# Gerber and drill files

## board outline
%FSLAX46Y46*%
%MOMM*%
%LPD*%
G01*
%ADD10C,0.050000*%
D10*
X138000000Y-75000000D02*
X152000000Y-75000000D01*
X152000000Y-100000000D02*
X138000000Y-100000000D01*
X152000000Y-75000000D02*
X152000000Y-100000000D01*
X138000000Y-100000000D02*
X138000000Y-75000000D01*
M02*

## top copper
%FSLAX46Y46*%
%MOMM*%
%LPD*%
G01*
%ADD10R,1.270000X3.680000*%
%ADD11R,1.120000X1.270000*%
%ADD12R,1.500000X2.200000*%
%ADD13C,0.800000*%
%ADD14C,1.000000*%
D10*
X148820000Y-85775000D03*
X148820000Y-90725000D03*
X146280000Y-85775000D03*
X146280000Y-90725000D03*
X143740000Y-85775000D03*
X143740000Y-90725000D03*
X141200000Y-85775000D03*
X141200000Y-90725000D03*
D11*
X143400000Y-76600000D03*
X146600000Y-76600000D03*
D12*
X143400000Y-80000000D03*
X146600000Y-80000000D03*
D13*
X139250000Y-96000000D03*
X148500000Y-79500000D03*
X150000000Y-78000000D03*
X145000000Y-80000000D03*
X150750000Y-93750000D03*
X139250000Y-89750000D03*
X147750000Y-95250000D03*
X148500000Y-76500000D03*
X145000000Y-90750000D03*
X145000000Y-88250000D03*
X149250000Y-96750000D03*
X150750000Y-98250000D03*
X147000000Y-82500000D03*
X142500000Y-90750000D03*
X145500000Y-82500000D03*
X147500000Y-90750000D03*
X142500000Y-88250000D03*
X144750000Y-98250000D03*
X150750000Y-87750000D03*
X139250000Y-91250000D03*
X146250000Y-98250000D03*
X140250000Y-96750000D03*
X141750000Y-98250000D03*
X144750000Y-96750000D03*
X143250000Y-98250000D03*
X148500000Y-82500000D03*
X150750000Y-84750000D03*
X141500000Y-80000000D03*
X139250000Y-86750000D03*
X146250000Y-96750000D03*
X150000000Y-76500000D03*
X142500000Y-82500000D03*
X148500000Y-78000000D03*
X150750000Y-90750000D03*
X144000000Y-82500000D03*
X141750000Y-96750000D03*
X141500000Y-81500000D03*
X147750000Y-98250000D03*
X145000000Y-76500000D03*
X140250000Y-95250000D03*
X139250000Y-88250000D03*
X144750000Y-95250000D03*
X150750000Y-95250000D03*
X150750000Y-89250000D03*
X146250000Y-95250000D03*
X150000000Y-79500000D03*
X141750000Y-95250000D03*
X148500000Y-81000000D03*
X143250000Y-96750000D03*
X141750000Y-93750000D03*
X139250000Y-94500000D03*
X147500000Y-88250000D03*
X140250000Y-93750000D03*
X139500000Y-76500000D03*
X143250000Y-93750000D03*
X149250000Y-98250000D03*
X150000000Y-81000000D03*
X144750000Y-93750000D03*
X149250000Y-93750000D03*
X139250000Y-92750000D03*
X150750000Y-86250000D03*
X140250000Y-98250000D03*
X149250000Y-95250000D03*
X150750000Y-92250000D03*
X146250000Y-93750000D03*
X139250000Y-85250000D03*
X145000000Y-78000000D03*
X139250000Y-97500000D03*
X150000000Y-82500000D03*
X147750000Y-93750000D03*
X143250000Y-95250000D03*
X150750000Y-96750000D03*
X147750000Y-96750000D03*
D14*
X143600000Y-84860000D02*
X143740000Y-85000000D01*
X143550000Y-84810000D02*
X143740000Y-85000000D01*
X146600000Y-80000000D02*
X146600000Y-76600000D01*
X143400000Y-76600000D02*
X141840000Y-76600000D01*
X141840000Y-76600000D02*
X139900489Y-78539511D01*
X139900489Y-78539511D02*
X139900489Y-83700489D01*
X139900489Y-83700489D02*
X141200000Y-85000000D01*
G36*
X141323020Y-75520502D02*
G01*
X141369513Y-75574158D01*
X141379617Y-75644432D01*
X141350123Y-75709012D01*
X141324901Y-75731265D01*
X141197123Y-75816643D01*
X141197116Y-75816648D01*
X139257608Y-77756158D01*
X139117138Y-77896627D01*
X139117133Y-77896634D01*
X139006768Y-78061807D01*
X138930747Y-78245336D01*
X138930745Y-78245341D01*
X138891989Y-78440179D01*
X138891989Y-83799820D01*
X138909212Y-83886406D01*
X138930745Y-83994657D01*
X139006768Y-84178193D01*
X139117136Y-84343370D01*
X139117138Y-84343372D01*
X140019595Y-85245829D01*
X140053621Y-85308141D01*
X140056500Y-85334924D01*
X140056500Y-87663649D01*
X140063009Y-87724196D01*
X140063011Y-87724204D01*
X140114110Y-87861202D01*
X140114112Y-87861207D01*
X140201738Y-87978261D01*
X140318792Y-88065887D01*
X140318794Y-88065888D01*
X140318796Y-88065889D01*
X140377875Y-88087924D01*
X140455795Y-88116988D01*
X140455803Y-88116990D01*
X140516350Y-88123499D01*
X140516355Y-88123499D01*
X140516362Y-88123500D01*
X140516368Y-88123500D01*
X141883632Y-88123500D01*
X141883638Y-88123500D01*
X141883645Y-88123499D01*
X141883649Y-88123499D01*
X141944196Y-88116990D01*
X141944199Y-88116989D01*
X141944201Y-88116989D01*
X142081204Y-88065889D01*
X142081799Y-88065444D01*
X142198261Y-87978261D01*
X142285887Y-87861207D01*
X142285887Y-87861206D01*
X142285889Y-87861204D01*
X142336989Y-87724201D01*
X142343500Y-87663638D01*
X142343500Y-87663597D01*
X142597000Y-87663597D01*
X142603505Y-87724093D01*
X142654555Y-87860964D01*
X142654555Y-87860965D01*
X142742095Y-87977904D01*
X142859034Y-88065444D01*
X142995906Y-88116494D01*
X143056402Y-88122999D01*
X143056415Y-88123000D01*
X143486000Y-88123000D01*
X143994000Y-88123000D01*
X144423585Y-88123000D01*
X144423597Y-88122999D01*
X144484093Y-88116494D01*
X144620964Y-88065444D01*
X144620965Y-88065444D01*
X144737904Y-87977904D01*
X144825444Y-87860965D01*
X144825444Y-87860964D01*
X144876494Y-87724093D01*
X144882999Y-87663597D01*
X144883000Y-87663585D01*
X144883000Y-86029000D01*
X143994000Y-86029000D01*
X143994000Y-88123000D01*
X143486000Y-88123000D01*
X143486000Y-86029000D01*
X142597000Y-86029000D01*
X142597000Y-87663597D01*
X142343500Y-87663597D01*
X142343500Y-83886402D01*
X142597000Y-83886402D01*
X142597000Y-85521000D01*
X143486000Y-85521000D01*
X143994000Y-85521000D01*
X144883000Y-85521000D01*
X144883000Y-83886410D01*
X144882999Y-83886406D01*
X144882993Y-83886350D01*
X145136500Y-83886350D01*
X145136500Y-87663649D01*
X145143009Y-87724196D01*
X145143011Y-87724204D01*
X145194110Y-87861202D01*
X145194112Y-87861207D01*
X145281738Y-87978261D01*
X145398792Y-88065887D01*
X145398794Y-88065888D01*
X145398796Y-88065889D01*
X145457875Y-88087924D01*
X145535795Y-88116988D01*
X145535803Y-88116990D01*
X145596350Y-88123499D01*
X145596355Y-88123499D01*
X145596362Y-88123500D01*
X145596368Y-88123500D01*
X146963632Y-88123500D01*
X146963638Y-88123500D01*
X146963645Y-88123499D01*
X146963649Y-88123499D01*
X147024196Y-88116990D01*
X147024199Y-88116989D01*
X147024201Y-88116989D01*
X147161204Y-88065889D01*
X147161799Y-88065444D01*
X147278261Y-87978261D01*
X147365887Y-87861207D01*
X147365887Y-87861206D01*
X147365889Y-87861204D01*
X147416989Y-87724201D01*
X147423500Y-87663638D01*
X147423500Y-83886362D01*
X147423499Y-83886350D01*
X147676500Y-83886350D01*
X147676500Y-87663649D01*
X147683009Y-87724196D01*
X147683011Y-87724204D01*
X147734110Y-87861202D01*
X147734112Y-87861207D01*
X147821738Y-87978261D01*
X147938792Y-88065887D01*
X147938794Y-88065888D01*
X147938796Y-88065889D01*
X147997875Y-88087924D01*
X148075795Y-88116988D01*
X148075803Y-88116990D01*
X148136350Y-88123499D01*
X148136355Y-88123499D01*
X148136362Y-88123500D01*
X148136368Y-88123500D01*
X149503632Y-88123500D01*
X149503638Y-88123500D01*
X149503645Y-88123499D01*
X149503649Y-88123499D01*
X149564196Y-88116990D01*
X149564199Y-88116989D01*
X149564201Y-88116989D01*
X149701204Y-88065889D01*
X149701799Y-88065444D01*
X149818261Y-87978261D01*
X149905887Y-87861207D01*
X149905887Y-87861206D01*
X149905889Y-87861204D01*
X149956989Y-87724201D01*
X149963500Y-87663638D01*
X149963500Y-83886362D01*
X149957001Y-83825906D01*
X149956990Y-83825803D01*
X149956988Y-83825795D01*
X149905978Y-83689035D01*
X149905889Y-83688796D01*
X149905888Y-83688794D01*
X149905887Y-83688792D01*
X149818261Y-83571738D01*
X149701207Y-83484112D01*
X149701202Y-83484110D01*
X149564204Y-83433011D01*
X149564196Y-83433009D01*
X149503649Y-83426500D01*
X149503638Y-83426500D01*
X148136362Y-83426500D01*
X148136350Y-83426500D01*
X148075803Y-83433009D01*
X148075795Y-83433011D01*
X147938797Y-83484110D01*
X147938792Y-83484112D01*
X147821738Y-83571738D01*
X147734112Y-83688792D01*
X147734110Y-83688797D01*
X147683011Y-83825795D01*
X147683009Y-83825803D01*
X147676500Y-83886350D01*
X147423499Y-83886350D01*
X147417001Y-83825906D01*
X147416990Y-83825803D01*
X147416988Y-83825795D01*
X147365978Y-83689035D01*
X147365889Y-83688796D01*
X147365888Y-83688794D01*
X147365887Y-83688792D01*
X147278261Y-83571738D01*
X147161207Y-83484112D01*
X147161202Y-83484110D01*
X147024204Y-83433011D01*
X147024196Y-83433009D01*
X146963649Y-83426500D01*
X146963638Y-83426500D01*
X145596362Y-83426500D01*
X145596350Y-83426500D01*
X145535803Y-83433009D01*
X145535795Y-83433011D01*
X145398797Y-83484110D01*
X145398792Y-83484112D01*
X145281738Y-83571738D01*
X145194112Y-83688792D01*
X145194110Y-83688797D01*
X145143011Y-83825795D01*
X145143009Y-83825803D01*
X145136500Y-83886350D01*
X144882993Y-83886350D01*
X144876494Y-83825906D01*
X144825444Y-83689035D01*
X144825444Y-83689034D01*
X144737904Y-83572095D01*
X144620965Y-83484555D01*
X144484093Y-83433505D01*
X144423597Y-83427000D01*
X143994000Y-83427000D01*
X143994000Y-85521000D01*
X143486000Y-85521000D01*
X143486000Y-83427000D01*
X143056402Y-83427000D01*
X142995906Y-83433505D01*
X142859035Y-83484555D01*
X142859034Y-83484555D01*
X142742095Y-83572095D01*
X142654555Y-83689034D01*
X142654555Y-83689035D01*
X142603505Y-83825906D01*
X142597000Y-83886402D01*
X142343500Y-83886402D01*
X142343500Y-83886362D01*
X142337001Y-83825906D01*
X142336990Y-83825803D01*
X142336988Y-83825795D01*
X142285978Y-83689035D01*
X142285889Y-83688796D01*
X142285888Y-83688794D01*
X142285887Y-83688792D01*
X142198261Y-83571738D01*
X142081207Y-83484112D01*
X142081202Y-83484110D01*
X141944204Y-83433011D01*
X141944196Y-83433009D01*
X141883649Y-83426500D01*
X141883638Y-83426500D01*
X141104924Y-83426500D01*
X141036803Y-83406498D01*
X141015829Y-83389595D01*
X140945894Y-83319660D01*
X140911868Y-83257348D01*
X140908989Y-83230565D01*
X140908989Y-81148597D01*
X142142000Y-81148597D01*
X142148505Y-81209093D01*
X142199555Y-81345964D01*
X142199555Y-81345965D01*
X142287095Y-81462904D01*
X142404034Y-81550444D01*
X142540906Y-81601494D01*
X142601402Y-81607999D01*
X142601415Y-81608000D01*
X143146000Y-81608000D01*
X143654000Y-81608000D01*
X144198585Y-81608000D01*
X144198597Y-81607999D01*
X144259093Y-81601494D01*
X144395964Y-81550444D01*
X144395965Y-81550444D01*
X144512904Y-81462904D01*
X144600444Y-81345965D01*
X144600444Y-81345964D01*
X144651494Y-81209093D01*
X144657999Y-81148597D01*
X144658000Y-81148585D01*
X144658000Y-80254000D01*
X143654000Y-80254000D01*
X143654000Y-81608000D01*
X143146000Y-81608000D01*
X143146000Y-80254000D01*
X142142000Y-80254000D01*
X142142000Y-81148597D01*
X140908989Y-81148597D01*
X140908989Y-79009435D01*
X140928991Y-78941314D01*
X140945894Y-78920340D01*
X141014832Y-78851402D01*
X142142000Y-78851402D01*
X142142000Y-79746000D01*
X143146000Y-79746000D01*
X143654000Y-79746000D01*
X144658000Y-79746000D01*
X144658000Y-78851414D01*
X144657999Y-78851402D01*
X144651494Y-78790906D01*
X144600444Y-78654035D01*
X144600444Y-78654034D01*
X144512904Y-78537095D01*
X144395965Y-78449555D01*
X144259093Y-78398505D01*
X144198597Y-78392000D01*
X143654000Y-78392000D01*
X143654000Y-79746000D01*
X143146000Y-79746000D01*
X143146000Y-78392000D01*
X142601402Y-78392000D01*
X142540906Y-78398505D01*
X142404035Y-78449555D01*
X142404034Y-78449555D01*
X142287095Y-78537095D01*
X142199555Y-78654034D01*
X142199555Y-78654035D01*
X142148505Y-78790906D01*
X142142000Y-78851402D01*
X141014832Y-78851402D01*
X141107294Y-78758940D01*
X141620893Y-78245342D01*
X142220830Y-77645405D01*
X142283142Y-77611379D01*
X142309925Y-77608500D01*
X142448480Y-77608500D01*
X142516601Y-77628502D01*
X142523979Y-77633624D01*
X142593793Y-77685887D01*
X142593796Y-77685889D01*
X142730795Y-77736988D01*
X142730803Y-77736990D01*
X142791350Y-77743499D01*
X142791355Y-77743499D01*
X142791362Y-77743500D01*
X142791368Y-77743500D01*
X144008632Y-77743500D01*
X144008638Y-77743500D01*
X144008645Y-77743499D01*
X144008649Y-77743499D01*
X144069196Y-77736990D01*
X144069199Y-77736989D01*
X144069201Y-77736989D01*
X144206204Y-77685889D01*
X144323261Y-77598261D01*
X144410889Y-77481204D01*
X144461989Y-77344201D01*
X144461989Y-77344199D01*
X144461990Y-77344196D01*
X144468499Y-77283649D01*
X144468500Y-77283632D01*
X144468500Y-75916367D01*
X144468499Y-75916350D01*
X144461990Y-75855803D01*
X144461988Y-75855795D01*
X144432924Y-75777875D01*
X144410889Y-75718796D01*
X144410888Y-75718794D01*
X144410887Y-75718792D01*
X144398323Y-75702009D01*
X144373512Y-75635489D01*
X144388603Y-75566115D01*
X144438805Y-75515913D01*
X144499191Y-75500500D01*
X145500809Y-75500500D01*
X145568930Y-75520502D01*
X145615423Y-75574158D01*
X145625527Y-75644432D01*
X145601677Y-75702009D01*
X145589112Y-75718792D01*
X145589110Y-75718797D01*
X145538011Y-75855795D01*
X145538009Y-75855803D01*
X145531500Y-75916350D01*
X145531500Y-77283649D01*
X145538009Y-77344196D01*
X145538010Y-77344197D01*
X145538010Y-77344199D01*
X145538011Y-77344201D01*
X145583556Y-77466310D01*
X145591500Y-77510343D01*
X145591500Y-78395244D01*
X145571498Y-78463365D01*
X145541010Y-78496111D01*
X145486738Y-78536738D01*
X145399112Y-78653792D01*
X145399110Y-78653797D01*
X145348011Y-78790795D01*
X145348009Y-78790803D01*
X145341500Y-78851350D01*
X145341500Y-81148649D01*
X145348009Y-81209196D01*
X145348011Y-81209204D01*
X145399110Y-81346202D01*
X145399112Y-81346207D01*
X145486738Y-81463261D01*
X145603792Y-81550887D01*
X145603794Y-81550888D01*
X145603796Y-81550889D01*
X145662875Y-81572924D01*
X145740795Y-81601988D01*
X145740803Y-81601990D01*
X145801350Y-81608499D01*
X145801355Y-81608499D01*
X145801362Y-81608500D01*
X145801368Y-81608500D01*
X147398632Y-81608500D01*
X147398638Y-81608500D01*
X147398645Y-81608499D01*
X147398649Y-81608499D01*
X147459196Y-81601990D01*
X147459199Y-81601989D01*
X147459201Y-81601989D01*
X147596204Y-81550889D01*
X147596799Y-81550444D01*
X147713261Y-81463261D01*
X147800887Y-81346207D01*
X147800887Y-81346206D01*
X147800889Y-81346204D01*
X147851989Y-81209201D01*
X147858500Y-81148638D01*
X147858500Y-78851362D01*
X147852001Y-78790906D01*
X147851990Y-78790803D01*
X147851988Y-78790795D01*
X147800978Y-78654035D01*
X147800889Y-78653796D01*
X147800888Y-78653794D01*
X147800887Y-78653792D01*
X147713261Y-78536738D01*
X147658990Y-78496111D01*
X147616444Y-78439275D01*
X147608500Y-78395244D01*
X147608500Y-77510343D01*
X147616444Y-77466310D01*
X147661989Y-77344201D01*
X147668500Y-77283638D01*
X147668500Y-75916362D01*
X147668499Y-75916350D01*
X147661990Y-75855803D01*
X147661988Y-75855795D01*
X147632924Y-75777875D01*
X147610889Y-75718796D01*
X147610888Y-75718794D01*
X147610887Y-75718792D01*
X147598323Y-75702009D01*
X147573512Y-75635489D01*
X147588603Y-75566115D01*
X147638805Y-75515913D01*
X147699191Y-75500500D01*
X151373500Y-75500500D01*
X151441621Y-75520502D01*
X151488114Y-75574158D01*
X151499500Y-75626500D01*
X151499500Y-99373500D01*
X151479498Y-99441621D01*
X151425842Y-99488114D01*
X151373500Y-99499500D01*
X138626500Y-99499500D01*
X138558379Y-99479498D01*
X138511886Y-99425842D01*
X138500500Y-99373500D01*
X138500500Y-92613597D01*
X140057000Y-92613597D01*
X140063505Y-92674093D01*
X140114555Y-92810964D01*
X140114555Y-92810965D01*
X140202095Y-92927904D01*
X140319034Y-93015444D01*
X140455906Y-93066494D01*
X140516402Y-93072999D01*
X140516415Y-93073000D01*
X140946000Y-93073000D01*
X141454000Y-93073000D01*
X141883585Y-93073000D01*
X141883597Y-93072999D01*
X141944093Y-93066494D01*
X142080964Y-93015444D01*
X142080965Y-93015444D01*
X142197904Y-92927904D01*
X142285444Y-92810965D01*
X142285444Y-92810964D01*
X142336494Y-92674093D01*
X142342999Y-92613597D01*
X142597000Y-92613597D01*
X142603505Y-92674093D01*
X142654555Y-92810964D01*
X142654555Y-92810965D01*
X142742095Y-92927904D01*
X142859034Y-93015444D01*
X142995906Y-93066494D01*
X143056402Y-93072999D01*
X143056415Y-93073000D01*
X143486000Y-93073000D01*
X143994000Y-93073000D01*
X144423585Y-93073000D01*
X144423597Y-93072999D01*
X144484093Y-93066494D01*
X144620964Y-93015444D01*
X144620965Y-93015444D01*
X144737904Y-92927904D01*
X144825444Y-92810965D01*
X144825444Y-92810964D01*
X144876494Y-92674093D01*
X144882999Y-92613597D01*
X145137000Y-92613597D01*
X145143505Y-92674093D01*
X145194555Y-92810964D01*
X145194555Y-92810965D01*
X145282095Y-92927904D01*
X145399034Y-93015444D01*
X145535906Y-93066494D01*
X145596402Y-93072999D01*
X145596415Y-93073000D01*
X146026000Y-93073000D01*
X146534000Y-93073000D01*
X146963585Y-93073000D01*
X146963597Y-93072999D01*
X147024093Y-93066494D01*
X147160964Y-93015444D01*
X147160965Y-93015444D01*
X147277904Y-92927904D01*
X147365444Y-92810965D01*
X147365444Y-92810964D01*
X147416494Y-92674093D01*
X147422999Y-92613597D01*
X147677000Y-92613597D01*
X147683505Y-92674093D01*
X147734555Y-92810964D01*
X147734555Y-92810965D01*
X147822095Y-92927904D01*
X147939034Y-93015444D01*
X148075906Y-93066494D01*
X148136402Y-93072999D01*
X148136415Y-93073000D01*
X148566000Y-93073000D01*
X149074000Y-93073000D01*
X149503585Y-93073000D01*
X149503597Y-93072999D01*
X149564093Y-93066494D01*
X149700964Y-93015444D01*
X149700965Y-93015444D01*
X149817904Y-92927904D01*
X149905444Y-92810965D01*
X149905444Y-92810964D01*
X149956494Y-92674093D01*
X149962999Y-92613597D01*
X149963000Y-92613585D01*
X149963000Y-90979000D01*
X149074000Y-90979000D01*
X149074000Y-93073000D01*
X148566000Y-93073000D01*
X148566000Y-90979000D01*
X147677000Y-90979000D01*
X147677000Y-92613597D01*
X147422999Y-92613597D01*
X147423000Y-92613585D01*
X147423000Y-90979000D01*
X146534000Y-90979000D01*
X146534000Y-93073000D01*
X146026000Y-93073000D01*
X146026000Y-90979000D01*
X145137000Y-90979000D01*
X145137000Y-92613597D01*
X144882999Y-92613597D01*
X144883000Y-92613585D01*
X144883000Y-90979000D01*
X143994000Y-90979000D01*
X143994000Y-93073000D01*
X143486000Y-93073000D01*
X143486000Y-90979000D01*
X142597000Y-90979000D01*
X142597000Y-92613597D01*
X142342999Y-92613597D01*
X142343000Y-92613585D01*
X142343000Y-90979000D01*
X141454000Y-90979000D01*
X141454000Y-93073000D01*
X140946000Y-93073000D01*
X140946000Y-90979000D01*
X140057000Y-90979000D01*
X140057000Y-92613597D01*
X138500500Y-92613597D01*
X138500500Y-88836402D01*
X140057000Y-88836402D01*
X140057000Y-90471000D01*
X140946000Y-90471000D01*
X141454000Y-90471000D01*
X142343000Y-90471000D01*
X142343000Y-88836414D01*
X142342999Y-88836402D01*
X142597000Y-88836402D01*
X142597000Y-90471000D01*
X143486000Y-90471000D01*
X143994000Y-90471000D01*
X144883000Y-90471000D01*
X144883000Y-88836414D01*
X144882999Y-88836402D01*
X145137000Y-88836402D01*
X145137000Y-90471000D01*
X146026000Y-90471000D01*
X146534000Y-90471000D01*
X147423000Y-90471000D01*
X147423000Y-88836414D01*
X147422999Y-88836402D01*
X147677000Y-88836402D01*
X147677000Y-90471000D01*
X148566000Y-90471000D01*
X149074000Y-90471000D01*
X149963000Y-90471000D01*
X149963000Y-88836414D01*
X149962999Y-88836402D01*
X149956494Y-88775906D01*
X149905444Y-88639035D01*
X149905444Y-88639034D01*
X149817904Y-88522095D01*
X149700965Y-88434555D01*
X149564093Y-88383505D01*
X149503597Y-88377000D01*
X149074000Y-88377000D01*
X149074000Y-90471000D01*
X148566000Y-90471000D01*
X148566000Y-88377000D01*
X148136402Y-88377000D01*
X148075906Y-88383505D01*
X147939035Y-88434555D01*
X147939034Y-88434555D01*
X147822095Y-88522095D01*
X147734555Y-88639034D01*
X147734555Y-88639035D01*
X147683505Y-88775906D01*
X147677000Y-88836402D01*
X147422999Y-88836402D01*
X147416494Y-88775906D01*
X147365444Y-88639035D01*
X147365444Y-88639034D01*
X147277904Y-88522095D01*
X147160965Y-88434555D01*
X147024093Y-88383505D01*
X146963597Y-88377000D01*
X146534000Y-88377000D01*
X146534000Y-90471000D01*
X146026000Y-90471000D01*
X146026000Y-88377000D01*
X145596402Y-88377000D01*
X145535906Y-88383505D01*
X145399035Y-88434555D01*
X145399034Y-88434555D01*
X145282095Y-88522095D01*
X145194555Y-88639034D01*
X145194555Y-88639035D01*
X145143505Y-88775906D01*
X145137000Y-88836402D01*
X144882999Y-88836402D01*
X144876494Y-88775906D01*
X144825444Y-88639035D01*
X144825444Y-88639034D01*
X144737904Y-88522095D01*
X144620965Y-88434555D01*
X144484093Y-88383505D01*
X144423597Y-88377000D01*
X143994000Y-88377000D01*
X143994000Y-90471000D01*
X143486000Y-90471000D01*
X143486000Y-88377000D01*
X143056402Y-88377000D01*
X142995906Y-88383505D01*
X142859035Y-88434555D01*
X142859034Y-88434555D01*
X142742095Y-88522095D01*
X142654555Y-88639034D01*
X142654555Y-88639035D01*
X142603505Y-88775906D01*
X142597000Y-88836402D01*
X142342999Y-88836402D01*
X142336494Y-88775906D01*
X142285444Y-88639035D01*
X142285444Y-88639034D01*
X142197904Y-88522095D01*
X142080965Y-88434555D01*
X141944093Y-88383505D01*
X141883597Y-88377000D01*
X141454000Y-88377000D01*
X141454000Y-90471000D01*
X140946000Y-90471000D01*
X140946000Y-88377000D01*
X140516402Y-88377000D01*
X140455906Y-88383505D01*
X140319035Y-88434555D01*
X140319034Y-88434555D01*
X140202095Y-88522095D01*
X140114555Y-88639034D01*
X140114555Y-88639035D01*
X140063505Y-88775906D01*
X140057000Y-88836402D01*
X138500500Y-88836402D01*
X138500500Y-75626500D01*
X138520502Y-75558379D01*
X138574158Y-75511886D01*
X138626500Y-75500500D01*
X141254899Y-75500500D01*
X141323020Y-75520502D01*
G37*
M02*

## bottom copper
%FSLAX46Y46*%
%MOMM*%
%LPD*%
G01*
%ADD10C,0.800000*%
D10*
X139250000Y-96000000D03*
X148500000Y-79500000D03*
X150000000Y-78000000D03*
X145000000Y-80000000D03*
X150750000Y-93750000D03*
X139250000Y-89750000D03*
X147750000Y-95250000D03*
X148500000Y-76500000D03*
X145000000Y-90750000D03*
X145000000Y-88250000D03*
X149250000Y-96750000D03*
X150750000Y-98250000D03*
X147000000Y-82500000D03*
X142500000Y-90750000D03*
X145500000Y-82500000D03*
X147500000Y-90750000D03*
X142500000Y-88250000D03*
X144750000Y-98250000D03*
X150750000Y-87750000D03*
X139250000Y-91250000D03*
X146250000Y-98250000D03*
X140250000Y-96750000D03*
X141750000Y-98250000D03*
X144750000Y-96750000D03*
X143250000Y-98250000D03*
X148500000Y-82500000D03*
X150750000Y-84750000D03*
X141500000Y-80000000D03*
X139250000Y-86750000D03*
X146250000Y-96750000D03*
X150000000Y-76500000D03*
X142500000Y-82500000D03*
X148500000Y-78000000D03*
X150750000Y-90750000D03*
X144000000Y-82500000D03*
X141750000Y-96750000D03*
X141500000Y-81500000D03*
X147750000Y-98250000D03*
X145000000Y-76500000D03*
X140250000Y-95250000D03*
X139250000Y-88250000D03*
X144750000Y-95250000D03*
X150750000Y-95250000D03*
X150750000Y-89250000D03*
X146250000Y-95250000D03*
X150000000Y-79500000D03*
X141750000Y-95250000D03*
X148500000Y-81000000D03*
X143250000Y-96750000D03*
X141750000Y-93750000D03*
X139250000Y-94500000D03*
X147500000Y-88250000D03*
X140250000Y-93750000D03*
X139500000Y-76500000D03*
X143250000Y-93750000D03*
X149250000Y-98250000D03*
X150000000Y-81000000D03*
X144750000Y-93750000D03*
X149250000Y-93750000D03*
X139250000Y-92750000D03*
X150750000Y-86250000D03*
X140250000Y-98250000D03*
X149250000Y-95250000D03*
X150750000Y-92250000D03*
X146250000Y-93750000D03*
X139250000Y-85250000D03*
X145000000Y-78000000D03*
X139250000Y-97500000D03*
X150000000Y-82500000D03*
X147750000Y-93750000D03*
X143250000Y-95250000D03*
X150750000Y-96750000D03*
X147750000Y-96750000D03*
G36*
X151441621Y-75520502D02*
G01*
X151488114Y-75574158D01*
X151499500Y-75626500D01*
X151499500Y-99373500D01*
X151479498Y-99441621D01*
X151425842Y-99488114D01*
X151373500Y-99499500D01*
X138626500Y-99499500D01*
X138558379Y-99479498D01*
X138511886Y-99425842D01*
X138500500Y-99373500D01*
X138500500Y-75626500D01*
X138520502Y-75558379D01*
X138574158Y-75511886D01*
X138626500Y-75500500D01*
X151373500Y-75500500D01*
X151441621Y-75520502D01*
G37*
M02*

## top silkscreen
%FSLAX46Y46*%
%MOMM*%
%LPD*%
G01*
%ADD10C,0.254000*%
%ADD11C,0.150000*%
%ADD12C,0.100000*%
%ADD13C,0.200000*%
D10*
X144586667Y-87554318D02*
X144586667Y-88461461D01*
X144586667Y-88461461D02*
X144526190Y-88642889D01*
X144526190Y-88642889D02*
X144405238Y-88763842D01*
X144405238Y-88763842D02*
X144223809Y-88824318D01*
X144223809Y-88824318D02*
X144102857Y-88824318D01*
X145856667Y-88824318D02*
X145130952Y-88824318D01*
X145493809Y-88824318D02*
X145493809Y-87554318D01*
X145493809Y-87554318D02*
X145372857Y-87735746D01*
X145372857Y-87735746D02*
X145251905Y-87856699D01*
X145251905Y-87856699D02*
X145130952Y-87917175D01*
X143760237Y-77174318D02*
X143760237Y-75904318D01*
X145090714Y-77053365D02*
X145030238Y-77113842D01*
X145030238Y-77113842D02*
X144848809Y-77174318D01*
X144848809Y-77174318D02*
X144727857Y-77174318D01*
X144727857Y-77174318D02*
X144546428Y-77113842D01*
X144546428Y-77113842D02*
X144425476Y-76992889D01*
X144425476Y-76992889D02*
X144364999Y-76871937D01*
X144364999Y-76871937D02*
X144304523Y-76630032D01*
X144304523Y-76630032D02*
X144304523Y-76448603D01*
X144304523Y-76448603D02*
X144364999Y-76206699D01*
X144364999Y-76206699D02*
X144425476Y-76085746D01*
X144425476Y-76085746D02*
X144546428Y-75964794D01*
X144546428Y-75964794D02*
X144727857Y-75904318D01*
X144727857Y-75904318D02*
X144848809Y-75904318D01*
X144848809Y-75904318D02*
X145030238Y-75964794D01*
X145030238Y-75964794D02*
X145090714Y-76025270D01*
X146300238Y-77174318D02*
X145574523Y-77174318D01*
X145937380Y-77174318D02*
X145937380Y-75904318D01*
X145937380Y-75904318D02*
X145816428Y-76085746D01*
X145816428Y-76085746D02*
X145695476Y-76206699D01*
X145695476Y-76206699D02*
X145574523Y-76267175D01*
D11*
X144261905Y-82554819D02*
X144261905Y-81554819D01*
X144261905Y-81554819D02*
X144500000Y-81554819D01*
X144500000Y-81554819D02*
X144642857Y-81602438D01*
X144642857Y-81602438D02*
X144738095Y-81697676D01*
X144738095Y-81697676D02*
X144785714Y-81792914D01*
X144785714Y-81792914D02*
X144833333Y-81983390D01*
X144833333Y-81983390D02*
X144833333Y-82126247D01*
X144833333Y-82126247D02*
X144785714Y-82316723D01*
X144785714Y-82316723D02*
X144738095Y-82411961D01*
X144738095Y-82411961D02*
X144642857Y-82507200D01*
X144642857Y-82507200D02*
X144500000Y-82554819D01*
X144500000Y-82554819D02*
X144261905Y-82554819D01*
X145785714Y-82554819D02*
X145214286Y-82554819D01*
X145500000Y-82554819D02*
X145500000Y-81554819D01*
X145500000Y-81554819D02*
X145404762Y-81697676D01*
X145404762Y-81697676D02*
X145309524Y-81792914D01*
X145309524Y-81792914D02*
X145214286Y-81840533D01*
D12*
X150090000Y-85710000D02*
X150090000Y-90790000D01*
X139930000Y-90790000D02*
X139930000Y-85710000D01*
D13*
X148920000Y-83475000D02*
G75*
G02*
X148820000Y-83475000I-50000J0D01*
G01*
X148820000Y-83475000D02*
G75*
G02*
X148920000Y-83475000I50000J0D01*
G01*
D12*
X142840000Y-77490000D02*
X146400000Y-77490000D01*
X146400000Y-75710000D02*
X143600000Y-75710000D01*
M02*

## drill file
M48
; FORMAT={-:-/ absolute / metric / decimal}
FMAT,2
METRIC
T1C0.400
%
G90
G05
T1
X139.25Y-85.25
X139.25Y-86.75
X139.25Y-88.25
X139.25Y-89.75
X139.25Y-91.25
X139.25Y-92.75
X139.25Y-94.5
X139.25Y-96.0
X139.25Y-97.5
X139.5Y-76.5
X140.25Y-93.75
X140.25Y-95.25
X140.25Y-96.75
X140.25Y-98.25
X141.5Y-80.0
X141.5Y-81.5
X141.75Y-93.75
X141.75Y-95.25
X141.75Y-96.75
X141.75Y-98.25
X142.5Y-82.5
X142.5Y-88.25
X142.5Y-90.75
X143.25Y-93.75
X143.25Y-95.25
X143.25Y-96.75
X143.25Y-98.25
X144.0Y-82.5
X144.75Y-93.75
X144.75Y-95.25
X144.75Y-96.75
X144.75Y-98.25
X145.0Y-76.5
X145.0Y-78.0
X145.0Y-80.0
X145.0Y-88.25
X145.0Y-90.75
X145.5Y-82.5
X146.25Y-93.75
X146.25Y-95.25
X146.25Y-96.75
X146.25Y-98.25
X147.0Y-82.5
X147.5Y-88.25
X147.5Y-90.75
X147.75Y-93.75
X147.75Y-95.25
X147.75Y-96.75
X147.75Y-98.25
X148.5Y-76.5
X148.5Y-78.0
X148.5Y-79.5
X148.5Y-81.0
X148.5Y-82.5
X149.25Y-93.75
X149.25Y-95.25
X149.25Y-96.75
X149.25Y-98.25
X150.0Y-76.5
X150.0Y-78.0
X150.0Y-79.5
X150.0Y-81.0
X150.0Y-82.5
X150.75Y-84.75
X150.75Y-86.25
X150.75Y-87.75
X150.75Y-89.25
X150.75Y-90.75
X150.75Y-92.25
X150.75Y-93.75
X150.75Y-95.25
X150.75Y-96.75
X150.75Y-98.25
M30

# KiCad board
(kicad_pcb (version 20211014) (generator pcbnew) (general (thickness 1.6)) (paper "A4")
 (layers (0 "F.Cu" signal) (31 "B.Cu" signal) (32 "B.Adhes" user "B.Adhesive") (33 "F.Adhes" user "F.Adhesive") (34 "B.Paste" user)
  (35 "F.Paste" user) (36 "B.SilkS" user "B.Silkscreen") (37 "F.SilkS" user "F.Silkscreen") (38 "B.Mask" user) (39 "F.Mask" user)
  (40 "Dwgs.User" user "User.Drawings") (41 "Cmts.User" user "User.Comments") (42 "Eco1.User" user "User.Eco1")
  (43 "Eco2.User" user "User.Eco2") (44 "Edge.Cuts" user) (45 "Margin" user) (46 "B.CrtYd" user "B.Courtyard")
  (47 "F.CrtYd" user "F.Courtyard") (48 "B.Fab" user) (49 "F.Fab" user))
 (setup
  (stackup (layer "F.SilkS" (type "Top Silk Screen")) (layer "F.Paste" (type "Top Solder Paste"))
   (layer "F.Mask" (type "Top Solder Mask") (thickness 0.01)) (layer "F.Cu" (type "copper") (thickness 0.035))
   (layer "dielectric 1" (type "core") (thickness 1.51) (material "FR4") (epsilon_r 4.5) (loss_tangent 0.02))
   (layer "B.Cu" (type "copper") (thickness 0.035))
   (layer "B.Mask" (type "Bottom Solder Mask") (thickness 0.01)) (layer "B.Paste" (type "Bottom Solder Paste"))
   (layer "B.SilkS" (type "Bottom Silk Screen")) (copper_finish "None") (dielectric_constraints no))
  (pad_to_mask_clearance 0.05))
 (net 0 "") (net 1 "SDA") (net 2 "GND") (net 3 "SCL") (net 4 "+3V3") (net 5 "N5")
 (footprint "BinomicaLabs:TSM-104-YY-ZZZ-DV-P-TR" (layer "F.Cu") (at 145.01 88.25)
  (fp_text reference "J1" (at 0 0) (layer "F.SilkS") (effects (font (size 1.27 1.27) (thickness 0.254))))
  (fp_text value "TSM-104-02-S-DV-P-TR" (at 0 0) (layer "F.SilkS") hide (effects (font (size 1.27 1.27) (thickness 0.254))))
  (fp_line (start 5.08 -2.54) (end 5.08 2.54) (layer "F.SilkS") (width 0.1))
  (fp_line (start -5.08 2.54) (end -5.08 -2.54) (layer "F.SilkS") (width 0.1))
  (fp_circle (center 3.86 -4.775) (end 3.86 -4.725) (layer "F.SilkS") (width 0.2) (fill none))
  (pad "1" smd rect locked (at 3.81 -2.475) (size 1.27 3.68) (layers "F.Cu" "F.Paste" "F.Mask") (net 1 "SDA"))
  (pad "2" smd rect locked (at 3.81 2.475) (size 1.27 3.68) (layers "F.Cu" "F.Paste" "F.Mask") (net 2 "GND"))
  (pad "3" smd rect locked (at 1.27 -2.475) (size 1.27 3.68) (layers "F.Cu" "F.Paste" "F.Mask") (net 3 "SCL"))
  (pad "4" smd rect locked (at 1.27 2.475) (size 1.27 3.68) (layers "F.Cu" "F.Paste" "F.Mask") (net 2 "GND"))
  (pad "5" smd rect locked (at -1.27 -2.475) (size 1.27 3.68) (layers "F.Cu" "F.Paste" "F.Mask") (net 2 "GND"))
  (pad "6" smd rect locked (at -1.27 2.475) (size 1.27 3.68) (layers "F.Cu" "F.Paste" "F.Mask") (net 2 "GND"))
  (pad "7" smd rect locked (at -3.81 -2.475) (size 1.27 3.68) (layers "F.Cu" "F.Paste" "F.Mask") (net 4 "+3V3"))
  (pad "8" smd rect locked (at -3.81 2.475) (size 1.27 3.68) (layers "F.Cu" "F.Paste" "F.Mask") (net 2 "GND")))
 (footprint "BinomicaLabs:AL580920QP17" (layer "F.Cu") (at 145 76.6 180)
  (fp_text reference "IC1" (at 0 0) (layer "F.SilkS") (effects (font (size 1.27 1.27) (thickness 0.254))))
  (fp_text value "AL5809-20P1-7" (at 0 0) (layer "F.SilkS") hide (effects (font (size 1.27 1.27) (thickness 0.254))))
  (fp_line (start 2.16 -0.89) (end -1.4 -0.89) (layer "F.SilkS") (width 0.1))
  (fp_line (start -1.4 0.89) (end 1.4 0.89) (layer "F.SilkS") (width 0.1))
  (pad "1" smd rect locked (at 1.6 0 180) (size 1.12 1.27) (layers "F.Cu" "F.Paste" "F.Mask") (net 4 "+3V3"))
  (pad "2" smd rect locked (at -1.6 0 180) (size 1.12 1.27) (layers "F.Cu" "F.Paste" "F.Mask") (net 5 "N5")))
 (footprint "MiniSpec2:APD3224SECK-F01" (layer "F.Cu") (at 145 80)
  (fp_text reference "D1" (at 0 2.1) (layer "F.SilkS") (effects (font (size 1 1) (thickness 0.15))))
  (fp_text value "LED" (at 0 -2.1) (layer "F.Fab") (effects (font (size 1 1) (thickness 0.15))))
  (pad "1" smd rect locked (at -1.6 0) (size 1.5 2.2) (layers "F.Cu" "F.Paste" "F.Mask") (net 2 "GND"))
  (pad "2" smd rect locked (at 1.6 0) (size 1.5 2.2) (layers "F.Cu" "F.Paste" "F.Mask") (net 5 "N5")))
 (gr_line (start 138 75) (end 152 75) (layer "Edge.Cuts") (width 0.05))
 (gr_line (start 152 100) (end 138 100) (layer "Edge.Cuts") (width 0.05))
 (gr_line (start 152 75) (end 152 100) (layer "Edge.Cuts") (width 0.05))
 (gr_line (start 138 100) (end 138 75) (layer "Edge.Cuts") (width 0.05))
 (segment (start 143.6 84.86) (end 143.74 85) (width 1) (layer "F.Cu") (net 2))
 (segment (start 143.55 84.81) (end 143.74 85) (width 1) (layer "F.Cu") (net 2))
 (via (at 139.25 96) (size 0.8) (drill 0.4) (layers "F.Cu" "B.Cu") (free) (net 2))
 (via (at 148.5 79.5) (size 0.8) (drill 0.4) (layers "F.Cu" "B.Cu") (free) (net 2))
 (via (at 150 78) (size 0.8) (drill 0.4) (layers "F.Cu" "B.Cu") (free) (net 2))
 (via (at 145 80) (size 0.8) (drill 0.4) (layers "F.Cu" "B.Cu") (free) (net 2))
 (via (at 150.75 93.75) (size 0.8) (drill 0.4) (layers "F.Cu" "B.Cu") (free) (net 2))
 (via (at 139.25 89.75) (size 0.8) (drill 0.4) (layers "F.Cu" "B.Cu") (free) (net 2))
 (via (at 147.75 95.25) (size 0.8) (drill 0.4) (layers "F.Cu" "B.Cu") (free) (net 2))
 (via (at 148.5 76.5) (size 0.8) (drill 0.4) (layers "F.Cu" "B.Cu") (free) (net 2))
 (via (at 145 90.75) (size 0.8) (drill 0.4) (layers "F.Cu" "B.Cu") (free) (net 2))
 (via (at 145 88.25) (size 0.8) (drill 0.4) (layers "F.Cu" "B.Cu") (free) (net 2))
 (via (at 149.25 96.75) (size 0.8) (drill 0.4) (layers "F.Cu" "B.Cu") (free) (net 2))
 (via (at 150.75 98.25) (size 0.8) (drill 0.4) (layers "F.Cu" "B.Cu") (free) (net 2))
 (via (at 147 82.5) (size 0.8) (drill 0.4) (layers "F.Cu" "B.Cu") (free) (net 2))
 (via (at 142.5 90.75) (size 0.8) (drill 0.4) (layers "F.Cu" "B.Cu") (free) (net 2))
 (via (at 145.5 82.5) (size 0.8) (drill 0.4) (layers "F.Cu" "B.Cu") (free) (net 2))
 (via (at 147.5 90.75) (size 0.8) (drill 0.4) (layers "F.Cu" "B.Cu") (free) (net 2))
 (via (at 142.5 88.25) (size 0.8) (drill 0.4) (layers "F.Cu" "B.Cu") (free) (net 2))
 (via (at 144.75 98.25) (size 0.8) (drill 0.4) (layers "F.Cu" "B.Cu") (free) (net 2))
 (via (at 150.75 87.75) (size 0.8) (drill 0.4) (layers "F.Cu" "B.Cu") (free) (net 2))
 (via (at 139.25 91.25) (size 0.8) (drill 0.4) (layers "F.Cu" "B.Cu") (free) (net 2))
 (via (at 146.25 98.25) (size 0.8) (drill 0.4) (layers "F.Cu" "B.Cu") (free) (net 2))
 (via (at 140.25 96.75) (size 0.8) (drill 0.4) (layers "F.Cu" "B.Cu") (free) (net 2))
 (via (at 141.75 98.25) (size 0.8) (drill 0.4) (layers "F.Cu" "B.Cu") (free) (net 2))
 (via (at 144.75 96.75) (size 0.8) (drill 0.4) (layers "F.Cu" "B.Cu") (free) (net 2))
 (via (at 143.25 98.25) (size 0.8) (drill 0.4) (layers "F.Cu" "B.Cu") (free) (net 2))
 (via (at 148.5 82.5) (size 0.8) (drill 0.4) (layers "F.Cu" "B.Cu") (free) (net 2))
 (via (at 150.75 84.75) (size 0.8) (drill 0.4) (layers "F.Cu" "B.Cu") (free) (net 2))
 (via (at 141.5 80) (size 0.8) (drill 0.4) (layers "F.Cu" "B.Cu") (free) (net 2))
 (via (at 139.25 86.75) (size 0.8) (drill 0.4) (layers "F.Cu" "B.Cu") (free) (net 2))
 (via (at 146.25 96.75) (size 0.8) (drill 0.4) (layers "F.Cu" "B.Cu") (free) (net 2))
 (via (at 150 76.5) (size 0.8) (drill 0.4) (layers "F.Cu" "B.Cu") (free) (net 2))
 (via (at 142.5 82.5) (size 0.8) (drill 0.4) (layers "F.Cu" "B.Cu") (free) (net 2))
 (via (at 148.5 78) (size 0.8) (drill 0.4) (layers "F.Cu" "B.Cu") (free) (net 2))
 (via (at 150.75 90.75) (size 0.8) (drill 0.4) (layers "F.Cu" "B.Cu") (free) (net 2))
 (via (at 144 82.5) (size 0.8) (drill 0.4) (layers "F.Cu" "B.Cu") (free) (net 2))
 (via (at 141.75 96.75) (size 0.8) (drill 0.4) (layers "F.Cu" "B.Cu") (free) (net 2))
 (via (at 141.5 81.5) (size 0.8) (drill 0.4) (layers "F.Cu" "B.Cu") (free) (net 2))
 (via (at 147.75 98.25) (size 0.8) (drill 0.4) (layers "F.Cu" "B.Cu") (free) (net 2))
 (via (at 145 76.5) (size 0.8) (drill 0.4) (layers "F.Cu" "B.Cu") (free) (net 2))
 (via (at 140.25 95.25) (size 0.8) (drill 0.4) (layers "F.Cu" "B.Cu") (free) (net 2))
 (via (at 139.25 88.25) (size 0.8) (drill 0.4) (layers "F.Cu" "B.Cu") (free) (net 2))
 (via (at 144.75 95.25) (size 0.8) (drill 0.4) (layers "F.Cu" "B.Cu") (free) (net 2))
 (via (at 150.75 95.25) (size 0.8) (drill 0.4) (layers "F.Cu" "B.Cu") (free) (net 2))
 (via (at 150.75 89.25) (size 0.8) (drill 0.4) (layers "F.Cu" "B.Cu") (free) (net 2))
 (via (at 146.25 95.25) (size 0.8) (drill 0.4) (layers "F.Cu" "B.Cu") (free) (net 2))
 (via (at 150 79.5) (size 0.8) (drill 0.4) (layers "F.Cu" "B.Cu") (free) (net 2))
 (via (at 141.75 95.25) (size 0.8) (drill 0.4) (layers "F.Cu" "B.Cu") (free) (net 2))
 (via (at 148.5 81) (size 0.8) (drill 0.4) (layers "F.Cu" "B.Cu") (free) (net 2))
 (via (at 143.25 96.75) (size 0.8) (drill 0.4) (layers "F.Cu" "B.Cu") (free) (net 2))
 (via (at 141.75 93.75) (size 0.8) (drill 0.4) (layers "F.Cu" "B.Cu") (free) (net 2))
 (via (at 139.25 94.5) (size 0.8) (drill 0.4) (layers "F.Cu" "B.Cu") (free) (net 2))
 (via (at 147.5 88.25) (size 0.8) (drill 0.4) (layers "F.Cu" "B.Cu") (free) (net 2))
 (via (at 140.25 93.75) (size 0.8) (drill 0.4) (layers "F.Cu" "B.Cu") (free) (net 2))
 (via (at 139.5 76.5) (size 0.8) (drill 0.4) (layers "F.Cu" "B.Cu") (free) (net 2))
 (via (at 143.25 93.75) (size 0.8) (drill 0.4) (layers "F.Cu" "B.Cu") (free) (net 2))
 (via (at 149.25 98.25) (size 0.8) (drill 0.4) (layers "F.Cu" "B.Cu") (free) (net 2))
 (via (at 150 81) (size 0.8) (drill 0.4) (layers "F.Cu" "B.Cu") (free) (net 2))
 (via (at 144.75 93.75) (size 0.8) (drill 0.4) (layers "F.Cu" "B.Cu") (free) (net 2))
 (via (at 149.25 93.75) (size 0.8) (drill 0.4) (layers "F.Cu" "B.Cu") (free) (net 2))
 (via (at 139.25 92.75) (size 0.8) (drill 0.4) (layers "F.Cu" "B.Cu") (free) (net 2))
 (via (at 150.75 86.25) (size 0.8) (drill 0.4) (layers "F.Cu" "B.Cu") (free) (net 2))
 (via (at 140.25 98.25) (size 0.8) (drill 0.4) (layers "F.Cu" "B.Cu") (free) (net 2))
 (via (at 149.25 95.25) (size 0.8) (drill 0.4) (layers "F.Cu" "B.Cu") (free) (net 2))
 (via (at 150.75 92.25) (size 0.8) (drill 0.4) (layers "F.Cu" "B.Cu") (free) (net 2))
 (via (at 146.25 93.75) (size 0.8) (drill 0.4) (layers "F.Cu" "B.Cu") (free) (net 2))
 (via (at 139.25 85.25) (size 0.8) (drill 0.4) (layers "F.Cu" "B.Cu") (free) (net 2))
 (via (at 145 78) (size 0.8) (drill 0.4) (layers "F.Cu" "B.Cu") (free) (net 2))
 (via (at 139.25 97.5) (size 0.8) (drill 0.4) (layers "F.Cu" "B.Cu") (free) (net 2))
 (via (at 150 82.5) (size 0.8) (drill 0.4) (layers "F.Cu" "B.Cu") (free) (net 2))
 (via (at 147.75 93.75) (size 0.8) (drill 0.4) (layers "F.Cu" "B.Cu") (free) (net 2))
 (via (at 143.25 95.25) (size 0.8) (drill 0.4) (layers "F.Cu" "B.Cu") (free) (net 2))
 (via (at 150.75 96.75) (size 0.8) (drill 0.4) (layers "F.Cu" "B.Cu") (free) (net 2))
 (via (at 147.75 96.75) (size 0.8) (drill 0.4) (layers "F.Cu" "B.Cu") (free) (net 2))
 (segment (start 146.6 80) (end 146.6 76.6) (width 1) (layer "F.Cu") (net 5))
 (segment (start 143.4 76.6) (end 141.84 76.6) (width 1) (layer "F.Cu") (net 4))
 (segment (start 141.84 76.6) (end 139.900489 78.539511) (width 1) (layer "F.Cu") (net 4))
 (segment (start 139.900489 78.539511) (end 139.900489 83.700489) (width 1) (layer "F.Cu") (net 4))
 (segment (start 139.900489 83.700489) (end 141.2 85) (width 1) (layer "F.Cu") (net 4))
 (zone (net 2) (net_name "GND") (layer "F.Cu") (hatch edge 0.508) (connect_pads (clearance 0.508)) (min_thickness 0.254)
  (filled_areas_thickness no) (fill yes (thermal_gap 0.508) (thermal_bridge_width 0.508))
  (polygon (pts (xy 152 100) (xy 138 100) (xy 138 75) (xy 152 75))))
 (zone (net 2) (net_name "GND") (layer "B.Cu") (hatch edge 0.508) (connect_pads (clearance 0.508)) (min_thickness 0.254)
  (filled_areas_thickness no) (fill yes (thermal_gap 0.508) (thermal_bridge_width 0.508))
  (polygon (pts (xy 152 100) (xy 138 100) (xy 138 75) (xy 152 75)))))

